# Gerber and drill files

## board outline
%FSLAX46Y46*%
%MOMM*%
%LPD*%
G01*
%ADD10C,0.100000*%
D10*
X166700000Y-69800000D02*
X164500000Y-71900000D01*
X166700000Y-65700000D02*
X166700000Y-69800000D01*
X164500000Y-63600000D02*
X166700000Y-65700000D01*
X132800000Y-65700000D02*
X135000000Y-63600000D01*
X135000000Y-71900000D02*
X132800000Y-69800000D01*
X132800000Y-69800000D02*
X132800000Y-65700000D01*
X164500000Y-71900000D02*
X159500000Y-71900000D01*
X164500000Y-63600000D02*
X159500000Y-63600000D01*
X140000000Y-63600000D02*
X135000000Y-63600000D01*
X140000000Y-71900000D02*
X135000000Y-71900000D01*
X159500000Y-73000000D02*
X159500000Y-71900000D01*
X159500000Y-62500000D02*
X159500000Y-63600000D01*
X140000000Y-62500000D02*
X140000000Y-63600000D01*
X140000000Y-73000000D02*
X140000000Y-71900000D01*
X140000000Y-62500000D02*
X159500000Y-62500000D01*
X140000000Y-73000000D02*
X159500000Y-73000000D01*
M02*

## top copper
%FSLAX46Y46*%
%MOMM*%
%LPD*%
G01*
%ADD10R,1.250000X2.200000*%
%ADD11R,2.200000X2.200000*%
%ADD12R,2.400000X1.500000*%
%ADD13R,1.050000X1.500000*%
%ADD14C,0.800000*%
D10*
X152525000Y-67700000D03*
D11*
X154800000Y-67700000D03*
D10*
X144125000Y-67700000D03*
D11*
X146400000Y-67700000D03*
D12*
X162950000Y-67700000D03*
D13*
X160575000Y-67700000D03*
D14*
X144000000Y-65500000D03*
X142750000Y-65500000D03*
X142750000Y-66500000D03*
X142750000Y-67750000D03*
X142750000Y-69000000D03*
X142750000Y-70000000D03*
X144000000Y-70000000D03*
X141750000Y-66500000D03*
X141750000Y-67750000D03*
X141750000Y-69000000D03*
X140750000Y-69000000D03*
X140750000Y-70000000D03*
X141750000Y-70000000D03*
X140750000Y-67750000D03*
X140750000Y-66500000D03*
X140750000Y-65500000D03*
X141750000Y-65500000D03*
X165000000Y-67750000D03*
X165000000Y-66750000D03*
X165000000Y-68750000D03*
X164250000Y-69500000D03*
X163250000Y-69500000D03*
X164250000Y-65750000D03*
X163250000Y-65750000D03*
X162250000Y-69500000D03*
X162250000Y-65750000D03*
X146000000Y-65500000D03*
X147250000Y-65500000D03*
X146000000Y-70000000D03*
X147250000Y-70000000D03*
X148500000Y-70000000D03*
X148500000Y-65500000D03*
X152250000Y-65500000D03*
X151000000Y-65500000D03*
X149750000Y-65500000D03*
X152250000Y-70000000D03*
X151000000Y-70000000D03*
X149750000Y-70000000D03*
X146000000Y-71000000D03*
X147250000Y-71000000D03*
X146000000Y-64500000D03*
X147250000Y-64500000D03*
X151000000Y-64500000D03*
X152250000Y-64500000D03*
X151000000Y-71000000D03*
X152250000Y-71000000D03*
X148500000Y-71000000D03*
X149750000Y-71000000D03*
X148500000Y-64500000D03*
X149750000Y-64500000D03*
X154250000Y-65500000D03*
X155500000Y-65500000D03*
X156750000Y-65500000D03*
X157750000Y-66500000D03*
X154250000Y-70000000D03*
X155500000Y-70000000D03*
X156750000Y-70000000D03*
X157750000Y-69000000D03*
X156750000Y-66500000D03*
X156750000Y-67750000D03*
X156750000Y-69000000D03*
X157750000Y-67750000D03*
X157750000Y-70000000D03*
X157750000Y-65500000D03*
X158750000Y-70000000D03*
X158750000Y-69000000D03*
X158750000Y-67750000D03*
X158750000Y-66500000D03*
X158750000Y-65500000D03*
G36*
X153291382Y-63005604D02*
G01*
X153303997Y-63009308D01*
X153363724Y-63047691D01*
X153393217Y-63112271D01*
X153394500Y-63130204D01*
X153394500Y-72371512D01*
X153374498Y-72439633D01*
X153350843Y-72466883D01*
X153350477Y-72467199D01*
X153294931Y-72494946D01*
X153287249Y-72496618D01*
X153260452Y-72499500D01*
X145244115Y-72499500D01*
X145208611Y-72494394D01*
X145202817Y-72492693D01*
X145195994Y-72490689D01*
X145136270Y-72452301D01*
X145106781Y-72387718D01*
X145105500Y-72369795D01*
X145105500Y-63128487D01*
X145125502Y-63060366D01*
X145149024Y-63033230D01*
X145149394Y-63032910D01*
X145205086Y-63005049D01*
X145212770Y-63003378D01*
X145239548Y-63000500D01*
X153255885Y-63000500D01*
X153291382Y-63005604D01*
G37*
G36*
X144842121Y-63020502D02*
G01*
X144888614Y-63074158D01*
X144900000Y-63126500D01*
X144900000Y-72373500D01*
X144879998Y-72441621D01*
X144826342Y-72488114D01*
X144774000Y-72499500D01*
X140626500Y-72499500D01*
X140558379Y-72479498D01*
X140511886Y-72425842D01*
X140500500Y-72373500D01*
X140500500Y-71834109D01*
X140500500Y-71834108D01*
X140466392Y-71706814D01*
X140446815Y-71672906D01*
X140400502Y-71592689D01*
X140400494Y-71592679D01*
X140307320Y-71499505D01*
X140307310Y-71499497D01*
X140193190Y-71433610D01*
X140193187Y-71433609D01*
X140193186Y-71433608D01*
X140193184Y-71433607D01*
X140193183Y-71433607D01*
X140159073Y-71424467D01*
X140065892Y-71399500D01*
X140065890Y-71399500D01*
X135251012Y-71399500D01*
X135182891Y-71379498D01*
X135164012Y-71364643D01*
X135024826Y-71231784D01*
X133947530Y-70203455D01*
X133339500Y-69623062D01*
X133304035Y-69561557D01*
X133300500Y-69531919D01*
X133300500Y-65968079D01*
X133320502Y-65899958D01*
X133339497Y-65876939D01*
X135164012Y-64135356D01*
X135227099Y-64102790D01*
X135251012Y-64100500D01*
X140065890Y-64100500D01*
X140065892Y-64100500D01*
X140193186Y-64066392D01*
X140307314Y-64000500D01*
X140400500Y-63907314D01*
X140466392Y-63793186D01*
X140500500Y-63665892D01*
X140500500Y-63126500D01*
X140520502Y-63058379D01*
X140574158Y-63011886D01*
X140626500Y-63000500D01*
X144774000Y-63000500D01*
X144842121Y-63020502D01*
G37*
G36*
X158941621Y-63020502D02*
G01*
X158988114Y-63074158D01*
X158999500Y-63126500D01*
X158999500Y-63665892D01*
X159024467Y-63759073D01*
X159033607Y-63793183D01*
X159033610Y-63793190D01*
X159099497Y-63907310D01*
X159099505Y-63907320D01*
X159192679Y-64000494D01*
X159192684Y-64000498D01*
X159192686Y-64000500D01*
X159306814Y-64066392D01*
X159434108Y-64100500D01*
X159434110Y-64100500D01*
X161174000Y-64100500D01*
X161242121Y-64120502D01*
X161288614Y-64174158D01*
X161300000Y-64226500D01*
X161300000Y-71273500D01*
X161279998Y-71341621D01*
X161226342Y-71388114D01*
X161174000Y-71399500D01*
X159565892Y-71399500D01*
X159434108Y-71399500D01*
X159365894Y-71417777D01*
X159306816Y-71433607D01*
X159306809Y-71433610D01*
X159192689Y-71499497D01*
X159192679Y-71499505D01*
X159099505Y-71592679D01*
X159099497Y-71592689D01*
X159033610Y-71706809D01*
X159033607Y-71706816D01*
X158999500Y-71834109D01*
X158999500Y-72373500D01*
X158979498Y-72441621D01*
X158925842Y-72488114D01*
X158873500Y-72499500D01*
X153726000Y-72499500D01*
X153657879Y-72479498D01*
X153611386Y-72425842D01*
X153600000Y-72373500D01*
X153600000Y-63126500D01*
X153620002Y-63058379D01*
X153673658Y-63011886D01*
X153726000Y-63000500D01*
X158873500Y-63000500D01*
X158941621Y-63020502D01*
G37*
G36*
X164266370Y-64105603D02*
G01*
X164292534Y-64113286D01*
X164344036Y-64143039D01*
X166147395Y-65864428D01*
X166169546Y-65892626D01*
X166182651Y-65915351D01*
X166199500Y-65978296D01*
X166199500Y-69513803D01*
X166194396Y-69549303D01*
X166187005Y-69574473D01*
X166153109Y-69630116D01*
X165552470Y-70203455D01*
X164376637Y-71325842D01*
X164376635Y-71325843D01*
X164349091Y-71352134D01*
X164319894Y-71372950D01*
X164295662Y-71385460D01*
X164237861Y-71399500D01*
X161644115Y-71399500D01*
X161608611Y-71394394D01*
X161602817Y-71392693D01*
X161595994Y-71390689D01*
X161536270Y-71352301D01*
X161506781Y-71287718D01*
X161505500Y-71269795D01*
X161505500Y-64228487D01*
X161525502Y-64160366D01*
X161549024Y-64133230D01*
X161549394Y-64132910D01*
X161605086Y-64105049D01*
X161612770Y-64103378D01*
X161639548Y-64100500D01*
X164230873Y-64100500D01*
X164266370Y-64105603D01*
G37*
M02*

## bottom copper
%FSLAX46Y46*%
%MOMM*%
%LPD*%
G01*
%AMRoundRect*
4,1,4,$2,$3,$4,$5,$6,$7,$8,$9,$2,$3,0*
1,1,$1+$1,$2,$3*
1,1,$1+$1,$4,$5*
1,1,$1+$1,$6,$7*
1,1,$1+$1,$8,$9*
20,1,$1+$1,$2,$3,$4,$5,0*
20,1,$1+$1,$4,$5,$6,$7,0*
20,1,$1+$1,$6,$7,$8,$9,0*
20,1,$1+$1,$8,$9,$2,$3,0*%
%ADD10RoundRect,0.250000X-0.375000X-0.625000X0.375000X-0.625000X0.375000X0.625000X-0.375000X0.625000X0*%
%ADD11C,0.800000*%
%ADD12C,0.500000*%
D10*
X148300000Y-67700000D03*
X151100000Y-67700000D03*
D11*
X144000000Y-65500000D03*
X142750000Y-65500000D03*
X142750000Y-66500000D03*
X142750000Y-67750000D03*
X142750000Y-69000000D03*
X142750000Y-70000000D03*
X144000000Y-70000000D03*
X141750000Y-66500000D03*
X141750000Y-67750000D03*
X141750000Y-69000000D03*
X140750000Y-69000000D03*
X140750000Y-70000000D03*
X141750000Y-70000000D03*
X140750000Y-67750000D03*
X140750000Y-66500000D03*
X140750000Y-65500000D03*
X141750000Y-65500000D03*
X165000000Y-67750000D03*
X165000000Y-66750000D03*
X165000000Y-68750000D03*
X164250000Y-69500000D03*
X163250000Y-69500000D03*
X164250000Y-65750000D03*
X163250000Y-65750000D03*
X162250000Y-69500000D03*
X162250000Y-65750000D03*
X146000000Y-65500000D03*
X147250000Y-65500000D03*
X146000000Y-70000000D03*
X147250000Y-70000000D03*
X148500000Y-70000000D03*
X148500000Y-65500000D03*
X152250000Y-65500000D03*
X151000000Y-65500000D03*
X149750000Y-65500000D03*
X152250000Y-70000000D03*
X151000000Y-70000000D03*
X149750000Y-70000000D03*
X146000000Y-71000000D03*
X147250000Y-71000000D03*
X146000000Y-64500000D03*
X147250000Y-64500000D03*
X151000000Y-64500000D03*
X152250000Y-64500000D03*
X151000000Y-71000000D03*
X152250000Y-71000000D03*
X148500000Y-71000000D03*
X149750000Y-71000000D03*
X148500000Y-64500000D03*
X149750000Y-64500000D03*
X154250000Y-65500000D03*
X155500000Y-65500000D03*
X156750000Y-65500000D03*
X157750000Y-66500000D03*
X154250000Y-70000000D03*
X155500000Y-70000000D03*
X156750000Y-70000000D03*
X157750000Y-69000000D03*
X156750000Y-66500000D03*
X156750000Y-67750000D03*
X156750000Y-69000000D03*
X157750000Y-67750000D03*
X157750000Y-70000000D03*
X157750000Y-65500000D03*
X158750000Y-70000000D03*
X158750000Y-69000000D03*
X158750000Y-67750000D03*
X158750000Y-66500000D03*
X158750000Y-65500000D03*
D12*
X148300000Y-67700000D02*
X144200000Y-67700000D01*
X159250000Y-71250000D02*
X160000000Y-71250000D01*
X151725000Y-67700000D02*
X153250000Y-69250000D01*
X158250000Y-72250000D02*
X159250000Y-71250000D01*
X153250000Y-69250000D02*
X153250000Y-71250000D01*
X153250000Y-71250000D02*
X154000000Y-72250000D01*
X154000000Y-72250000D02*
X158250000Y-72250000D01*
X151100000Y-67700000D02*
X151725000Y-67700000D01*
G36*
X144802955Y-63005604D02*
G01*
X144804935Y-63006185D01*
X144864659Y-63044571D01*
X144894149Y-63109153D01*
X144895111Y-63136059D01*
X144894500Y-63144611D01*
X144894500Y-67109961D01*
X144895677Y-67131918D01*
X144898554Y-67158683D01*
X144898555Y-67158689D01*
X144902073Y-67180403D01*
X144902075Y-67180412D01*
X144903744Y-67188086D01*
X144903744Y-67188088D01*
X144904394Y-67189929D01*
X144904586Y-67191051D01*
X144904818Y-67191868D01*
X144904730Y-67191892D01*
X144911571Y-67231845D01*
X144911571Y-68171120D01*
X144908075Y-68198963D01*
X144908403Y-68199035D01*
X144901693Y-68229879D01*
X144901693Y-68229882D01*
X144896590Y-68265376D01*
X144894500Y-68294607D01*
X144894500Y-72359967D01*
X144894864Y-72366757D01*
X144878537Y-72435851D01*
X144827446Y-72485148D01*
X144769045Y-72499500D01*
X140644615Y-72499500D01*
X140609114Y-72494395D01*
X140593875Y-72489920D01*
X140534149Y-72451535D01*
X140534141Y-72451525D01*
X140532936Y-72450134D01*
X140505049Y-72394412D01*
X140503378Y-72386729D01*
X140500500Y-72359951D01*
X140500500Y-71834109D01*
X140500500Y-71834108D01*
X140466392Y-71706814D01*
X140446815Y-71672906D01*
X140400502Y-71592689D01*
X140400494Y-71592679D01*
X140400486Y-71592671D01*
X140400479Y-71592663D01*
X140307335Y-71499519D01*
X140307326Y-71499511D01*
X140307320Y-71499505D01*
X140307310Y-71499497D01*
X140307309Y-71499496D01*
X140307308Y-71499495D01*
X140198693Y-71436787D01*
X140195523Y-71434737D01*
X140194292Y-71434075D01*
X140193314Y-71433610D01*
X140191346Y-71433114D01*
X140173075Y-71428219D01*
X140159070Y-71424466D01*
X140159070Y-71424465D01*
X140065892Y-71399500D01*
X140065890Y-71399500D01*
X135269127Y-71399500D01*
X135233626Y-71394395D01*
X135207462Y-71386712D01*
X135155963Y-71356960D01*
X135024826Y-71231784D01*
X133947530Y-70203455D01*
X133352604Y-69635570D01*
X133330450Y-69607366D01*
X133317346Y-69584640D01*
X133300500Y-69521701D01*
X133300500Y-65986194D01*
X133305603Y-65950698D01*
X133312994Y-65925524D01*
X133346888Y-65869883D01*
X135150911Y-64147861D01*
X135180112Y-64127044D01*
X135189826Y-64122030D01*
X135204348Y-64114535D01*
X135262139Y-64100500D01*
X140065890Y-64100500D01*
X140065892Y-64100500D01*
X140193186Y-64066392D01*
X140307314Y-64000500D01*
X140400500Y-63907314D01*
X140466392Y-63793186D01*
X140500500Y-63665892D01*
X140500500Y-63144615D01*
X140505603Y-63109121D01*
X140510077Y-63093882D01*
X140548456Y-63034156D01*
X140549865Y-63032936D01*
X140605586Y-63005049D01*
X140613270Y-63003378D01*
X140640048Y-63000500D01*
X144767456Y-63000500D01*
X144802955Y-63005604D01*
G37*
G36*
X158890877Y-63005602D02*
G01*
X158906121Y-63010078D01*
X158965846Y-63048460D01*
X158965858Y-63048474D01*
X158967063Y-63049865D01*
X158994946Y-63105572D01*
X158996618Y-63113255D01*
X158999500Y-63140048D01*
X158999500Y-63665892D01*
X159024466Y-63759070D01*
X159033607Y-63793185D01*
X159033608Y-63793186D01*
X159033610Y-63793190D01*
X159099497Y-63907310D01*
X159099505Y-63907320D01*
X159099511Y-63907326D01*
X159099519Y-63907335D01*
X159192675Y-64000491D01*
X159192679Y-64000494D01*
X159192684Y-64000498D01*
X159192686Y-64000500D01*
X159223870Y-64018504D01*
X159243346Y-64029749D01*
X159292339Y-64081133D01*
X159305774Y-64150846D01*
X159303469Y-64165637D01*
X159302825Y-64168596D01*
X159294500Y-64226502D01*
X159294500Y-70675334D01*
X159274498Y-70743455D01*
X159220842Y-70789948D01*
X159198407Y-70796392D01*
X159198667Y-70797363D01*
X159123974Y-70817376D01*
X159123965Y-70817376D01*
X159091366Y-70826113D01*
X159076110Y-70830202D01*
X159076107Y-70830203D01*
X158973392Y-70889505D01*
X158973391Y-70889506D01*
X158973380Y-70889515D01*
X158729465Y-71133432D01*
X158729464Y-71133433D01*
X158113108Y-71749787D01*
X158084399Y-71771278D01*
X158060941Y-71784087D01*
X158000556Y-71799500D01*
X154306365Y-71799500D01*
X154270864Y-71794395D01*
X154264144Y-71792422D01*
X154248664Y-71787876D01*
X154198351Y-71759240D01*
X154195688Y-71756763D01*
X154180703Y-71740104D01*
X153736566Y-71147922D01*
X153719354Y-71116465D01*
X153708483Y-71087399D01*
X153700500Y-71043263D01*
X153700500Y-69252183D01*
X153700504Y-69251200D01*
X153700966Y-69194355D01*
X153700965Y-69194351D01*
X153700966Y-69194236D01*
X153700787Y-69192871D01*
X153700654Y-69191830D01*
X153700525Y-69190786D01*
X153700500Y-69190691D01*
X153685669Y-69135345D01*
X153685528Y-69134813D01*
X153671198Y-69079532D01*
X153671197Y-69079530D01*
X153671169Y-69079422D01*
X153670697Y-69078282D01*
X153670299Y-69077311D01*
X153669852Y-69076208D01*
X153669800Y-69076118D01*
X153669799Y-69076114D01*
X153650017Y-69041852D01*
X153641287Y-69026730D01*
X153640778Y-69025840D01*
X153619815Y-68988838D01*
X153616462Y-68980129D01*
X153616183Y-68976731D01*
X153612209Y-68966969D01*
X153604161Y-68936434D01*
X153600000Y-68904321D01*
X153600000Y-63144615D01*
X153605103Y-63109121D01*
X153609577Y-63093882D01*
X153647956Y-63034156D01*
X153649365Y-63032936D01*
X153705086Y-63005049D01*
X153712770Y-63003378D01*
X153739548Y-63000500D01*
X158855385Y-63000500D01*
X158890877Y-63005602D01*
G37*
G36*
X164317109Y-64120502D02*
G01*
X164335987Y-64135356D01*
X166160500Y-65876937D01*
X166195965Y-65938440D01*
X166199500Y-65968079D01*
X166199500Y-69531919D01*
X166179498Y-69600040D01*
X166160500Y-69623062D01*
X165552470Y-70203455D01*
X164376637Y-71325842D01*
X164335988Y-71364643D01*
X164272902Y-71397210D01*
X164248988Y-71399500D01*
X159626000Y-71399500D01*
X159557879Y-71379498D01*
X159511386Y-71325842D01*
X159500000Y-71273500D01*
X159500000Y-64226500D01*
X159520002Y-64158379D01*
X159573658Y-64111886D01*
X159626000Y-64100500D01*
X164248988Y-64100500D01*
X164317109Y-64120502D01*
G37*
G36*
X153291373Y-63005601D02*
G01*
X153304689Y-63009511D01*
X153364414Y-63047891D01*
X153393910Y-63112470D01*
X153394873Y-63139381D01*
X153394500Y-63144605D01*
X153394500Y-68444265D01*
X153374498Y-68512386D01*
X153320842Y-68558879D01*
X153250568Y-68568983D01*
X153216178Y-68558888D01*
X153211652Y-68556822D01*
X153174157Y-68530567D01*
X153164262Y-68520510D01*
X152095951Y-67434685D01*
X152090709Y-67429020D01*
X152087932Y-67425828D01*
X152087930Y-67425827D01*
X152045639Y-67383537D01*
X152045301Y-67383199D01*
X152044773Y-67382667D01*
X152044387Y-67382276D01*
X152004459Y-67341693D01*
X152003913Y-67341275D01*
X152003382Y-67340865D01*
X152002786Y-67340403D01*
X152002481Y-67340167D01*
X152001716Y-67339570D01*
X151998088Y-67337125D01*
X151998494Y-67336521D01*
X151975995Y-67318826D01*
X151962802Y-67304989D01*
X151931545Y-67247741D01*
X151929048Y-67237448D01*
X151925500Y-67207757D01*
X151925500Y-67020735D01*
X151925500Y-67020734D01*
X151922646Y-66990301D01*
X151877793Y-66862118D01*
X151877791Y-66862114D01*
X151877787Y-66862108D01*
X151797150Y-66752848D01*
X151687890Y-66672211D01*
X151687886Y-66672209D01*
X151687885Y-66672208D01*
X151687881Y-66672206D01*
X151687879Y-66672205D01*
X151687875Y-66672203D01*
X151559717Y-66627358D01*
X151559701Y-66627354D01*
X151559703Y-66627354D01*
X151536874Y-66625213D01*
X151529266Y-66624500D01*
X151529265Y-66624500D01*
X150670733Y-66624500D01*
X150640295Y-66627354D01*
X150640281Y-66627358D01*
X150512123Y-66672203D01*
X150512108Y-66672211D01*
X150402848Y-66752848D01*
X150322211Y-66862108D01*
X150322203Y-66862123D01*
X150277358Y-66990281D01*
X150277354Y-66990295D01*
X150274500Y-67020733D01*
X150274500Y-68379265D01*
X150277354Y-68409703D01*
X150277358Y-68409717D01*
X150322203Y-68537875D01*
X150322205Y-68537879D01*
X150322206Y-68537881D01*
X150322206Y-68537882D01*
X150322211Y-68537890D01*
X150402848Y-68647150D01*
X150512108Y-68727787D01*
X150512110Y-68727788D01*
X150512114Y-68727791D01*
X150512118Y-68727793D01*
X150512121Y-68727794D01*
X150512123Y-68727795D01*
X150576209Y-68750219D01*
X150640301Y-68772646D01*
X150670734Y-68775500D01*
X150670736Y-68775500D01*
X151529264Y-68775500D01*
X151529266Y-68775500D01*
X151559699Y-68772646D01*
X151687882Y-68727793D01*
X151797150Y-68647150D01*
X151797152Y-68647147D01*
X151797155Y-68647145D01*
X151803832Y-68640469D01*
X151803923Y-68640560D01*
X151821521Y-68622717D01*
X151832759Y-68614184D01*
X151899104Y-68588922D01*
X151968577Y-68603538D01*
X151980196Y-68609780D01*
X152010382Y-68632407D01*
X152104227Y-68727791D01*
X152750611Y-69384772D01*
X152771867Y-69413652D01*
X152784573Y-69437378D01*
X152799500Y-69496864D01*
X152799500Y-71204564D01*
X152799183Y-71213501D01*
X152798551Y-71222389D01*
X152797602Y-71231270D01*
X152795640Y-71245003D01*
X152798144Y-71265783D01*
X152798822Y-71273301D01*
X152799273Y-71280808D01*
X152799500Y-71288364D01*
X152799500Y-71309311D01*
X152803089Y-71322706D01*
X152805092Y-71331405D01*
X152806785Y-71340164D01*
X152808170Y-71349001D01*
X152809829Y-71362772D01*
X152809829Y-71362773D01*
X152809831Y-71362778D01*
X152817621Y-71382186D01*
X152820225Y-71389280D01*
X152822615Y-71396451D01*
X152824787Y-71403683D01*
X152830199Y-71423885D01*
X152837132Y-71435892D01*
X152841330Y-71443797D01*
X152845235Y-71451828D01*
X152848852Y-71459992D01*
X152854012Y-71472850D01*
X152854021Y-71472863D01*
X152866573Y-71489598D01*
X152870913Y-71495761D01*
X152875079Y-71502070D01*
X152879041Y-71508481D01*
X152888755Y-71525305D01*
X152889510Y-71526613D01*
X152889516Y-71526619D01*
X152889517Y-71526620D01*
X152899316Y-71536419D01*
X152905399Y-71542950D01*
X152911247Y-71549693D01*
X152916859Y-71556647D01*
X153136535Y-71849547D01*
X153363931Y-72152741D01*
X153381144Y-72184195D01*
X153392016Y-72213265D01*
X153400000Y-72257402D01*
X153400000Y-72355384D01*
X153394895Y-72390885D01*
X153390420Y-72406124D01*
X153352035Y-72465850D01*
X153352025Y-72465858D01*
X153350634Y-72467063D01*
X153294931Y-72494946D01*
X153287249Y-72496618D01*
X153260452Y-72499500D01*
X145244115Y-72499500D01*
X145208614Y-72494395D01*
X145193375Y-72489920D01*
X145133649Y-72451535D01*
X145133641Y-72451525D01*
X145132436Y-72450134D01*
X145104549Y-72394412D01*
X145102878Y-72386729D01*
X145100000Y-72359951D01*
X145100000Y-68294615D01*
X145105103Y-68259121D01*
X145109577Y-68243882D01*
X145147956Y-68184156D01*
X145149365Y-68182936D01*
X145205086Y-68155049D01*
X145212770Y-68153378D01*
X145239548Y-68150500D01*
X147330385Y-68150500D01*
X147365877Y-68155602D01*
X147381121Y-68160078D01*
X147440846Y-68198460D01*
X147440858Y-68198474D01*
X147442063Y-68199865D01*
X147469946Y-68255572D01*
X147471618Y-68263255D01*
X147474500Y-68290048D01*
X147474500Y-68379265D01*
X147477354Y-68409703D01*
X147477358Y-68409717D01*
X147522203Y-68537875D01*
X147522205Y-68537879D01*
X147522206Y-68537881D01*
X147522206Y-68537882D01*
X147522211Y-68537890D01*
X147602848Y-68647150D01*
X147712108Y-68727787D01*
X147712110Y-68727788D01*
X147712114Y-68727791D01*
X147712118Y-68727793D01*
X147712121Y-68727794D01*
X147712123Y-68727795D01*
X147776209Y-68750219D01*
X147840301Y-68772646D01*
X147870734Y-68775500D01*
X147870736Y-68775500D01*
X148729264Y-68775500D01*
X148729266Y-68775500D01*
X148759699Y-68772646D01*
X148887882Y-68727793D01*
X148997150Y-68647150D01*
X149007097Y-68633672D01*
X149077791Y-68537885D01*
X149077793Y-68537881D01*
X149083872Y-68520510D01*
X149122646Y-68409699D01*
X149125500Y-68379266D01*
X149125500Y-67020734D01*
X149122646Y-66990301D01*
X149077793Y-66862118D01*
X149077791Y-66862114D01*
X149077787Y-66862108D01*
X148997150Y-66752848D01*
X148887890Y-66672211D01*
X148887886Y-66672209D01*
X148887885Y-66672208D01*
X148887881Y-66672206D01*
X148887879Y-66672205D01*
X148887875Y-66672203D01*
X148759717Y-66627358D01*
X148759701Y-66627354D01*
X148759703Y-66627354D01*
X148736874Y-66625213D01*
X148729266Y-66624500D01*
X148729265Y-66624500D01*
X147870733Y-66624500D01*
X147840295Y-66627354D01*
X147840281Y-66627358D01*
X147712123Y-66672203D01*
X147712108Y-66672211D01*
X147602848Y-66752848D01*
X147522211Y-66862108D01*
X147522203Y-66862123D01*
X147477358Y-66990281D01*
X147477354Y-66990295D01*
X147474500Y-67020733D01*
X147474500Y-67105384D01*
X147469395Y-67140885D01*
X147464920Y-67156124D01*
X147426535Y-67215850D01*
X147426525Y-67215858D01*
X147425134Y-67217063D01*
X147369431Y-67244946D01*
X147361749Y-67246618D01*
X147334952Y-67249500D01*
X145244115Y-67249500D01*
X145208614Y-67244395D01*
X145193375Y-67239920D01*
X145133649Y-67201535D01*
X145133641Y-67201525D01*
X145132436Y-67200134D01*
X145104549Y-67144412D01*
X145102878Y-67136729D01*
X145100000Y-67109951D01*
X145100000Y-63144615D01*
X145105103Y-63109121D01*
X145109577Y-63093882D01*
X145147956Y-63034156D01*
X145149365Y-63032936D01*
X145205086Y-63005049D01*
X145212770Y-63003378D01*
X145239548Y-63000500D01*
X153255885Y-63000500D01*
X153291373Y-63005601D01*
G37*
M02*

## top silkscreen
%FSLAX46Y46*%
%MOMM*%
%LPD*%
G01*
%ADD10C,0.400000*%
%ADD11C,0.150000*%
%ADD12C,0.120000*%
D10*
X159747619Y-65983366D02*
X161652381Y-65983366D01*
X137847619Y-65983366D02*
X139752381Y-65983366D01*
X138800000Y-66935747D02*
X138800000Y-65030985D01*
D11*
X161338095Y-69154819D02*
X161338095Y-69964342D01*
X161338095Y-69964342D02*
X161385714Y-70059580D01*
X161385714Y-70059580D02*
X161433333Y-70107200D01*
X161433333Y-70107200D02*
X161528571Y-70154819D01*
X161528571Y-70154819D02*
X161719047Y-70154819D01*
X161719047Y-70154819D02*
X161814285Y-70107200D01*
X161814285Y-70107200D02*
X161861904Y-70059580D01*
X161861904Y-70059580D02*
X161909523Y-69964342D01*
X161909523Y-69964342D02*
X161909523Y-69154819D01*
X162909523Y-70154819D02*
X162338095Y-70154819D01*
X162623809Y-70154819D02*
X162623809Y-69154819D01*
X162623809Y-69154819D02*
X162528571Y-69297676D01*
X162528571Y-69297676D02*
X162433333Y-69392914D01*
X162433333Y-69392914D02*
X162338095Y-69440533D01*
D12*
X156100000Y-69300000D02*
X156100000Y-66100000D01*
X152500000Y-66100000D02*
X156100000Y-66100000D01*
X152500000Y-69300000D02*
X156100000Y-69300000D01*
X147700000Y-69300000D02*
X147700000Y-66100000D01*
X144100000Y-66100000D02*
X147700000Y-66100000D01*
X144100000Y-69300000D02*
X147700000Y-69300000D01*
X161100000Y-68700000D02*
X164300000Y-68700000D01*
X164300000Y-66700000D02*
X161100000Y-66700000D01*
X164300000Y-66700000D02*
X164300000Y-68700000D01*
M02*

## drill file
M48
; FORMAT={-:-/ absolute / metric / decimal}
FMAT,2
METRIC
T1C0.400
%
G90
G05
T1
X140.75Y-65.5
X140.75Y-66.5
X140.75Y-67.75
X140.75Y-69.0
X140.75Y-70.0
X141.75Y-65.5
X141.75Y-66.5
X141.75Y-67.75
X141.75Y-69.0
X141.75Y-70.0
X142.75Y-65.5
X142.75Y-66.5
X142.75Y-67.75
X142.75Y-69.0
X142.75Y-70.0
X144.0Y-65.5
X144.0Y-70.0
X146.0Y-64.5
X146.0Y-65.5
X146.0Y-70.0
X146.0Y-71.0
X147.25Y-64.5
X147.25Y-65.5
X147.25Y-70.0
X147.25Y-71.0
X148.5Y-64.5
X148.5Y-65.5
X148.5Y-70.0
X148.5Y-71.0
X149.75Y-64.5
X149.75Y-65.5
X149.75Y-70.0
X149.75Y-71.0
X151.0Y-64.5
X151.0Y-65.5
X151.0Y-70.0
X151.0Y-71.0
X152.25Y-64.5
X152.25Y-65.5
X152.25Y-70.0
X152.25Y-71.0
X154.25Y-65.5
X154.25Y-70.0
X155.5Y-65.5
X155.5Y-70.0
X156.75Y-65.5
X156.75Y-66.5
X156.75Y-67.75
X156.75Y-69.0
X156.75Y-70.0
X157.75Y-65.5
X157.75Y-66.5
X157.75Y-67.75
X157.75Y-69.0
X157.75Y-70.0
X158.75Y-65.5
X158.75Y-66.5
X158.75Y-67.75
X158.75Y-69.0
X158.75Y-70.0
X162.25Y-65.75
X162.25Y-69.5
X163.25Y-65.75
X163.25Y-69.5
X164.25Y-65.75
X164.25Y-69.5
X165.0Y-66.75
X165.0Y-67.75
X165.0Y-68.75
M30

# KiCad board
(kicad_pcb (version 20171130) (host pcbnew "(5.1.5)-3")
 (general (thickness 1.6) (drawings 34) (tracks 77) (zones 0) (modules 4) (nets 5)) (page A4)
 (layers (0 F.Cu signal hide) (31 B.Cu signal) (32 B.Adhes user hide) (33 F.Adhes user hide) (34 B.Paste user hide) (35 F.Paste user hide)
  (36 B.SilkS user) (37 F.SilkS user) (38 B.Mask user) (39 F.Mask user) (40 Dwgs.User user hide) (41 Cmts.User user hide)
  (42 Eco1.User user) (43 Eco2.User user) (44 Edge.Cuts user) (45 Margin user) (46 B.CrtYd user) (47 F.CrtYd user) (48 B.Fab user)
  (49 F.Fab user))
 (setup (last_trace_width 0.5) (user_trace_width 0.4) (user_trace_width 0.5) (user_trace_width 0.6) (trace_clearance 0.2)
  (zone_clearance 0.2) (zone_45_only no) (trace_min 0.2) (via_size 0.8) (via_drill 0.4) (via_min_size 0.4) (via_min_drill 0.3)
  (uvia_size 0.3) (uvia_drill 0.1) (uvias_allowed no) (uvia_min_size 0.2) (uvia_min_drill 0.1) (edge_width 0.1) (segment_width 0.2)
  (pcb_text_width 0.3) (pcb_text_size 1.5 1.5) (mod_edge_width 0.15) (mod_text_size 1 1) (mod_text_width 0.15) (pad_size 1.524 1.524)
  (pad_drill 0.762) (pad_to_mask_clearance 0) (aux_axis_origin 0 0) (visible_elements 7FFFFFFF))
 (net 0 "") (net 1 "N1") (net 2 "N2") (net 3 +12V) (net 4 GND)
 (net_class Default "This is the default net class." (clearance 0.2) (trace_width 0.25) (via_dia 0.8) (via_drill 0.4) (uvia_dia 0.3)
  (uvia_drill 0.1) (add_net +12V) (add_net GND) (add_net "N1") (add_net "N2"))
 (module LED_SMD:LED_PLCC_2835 (layer F.Cu) (at 153.9 67.7 180)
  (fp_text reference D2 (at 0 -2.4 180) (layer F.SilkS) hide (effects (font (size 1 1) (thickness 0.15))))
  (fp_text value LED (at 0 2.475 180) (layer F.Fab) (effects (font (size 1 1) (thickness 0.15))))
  (fp_line (start -2.2 -1.6) (end -2.2 1.6) (layer F.SilkS) (width 0.12))
  (fp_line (start 1.4 1.6) (end -2.2 1.6) (layer F.SilkS) (width 0.12))
  (fp_line (start 1.4 -1.6) (end -2.2 -1.6) (layer F.SilkS) (width 0.12))
  (pad 2 smd rect (at 1.375 0 180) (size 1.25 2.2) (layers F.Cu F.Paste F.Mask) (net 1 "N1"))
  (pad 1 smd rect (at -0.9 0 180) (size 2.2 2.2) (layers F.Cu F.Paste F.Mask) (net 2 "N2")))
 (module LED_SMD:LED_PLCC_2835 (layer F.Cu) (at 145.5 67.7 180)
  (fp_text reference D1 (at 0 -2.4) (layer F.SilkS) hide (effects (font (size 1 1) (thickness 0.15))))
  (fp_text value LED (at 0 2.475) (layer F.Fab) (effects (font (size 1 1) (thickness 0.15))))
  (fp_line (start -2.2 -1.6) (end -2.2 1.6) (layer F.SilkS) (width 0.12))
  (fp_line (start 1.4 1.6) (end -2.2 1.6) (layer F.SilkS) (width 0.12))
  (fp_line (start 1.4 -1.6) (end -2.2 -1.6) (layer F.SilkS) (width 0.12))
  (pad 2 smd rect (at 1.375 0 180) (size 1.25 2.2) (layers F.Cu F.Paste F.Mask) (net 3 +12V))
  (pad 1 smd rect (at -0.9 0 180) (size 2.2 2.2) (layers F.Cu F.Paste F.Mask) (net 1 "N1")))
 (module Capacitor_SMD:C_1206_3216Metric (layer B.Cu) (at 149.7 67.7)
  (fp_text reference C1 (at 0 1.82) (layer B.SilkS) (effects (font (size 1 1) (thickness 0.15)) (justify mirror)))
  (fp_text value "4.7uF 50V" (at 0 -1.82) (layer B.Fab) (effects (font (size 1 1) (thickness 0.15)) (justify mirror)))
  (pad 1 smd roundrect (at -1.4 0) (size 1.25 1.75) (layers B.Cu B.Paste B.Mask) (roundrect_rratio 0.2) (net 3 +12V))
  (pad 2 smd roundrect (at 1.4 0) (size 1.25 1.75) (layers B.Cu B.Paste B.Mask) (roundrect_rratio 0.2) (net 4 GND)))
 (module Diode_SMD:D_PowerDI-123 (layer F.Cu) (at 162.1 67.7 180)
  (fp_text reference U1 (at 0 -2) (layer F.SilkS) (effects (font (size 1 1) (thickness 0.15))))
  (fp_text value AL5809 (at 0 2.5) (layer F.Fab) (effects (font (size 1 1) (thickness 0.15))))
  (fp_line (start 1 -1) (end -2.2 -1) (layer F.SilkS) (width 0.12))
  (fp_line (start -2.2 1) (end 1 1) (layer F.SilkS) (width 0.12))
  (fp_line (start -2.2 1) (end -2.2 -1) (layer F.SilkS) (width 0.12))
  (pad 1 smd rect (at -0.85 0) (size 2.4 1.5) (layers F.Cu F.Paste F.Mask) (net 4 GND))
  (pad 2 smd rect (at 1.525 0) (size 1.05 1.5) (layers F.Cu F.Paste F.Mask) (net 2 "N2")))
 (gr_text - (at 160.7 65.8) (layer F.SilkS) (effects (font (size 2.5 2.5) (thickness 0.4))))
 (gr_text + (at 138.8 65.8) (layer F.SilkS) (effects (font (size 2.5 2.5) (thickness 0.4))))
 (gr_line (start 166.7 69.8) (end 164.5 71.9) (layer Edge.Cuts) (width 0.1))
 (gr_line (start 166.7 65.7) (end 166.7 69.8) (layer Edge.Cuts) (width 0.1))
 (gr_line (start 164.5 63.6) (end 166.7 65.7) (layer Edge.Cuts) (width 0.1))
 (gr_line (start 132.8 65.7) (end 135 63.6) (layer Edge.Cuts) (width 0.1))
 (gr_line (start 135 71.9) (end 132.8 69.8) (layer Edge.Cuts) (width 0.1))
 (gr_line (start 132.8 69.8) (end 132.8 65.7) (layer Edge.Cuts) (width 0.1))
 (gr_line (start 164.5 71.9) (end 159.5 71.9) (layer Edge.Cuts) (width 0.1))
 (gr_line (start 164.5 63.6) (end 159.5 63.6) (layer Edge.Cuts) (width 0.1))
 (gr_line (start 140 63.6) (end 135 63.6) (layer Edge.Cuts) (width 0.1))
 (gr_line (start 140 71.9) (end 135 71.9) (layer Edge.Cuts) (width 0.1))
 (gr_line (start 159.5 73) (end 159.5 71.9) (layer Edge.Cuts) (width 0.1))
 (gr_line (start 159.5 62.5) (end 159.5 63.6) (layer Edge.Cuts) (width 0.1))
 (gr_line (start 140 62.5) (end 140 63.6) (layer Edge.Cuts) (width 0.1))
 (gr_line (start 140 73) (end 140 71.9) (layer Edge.Cuts) (width 0.1))
 (gr_line (start 140 62.5) (end 159.5 62.5) (layer Edge.Cuts) (width 0.1))
 (gr_line (start 140 73) (end 159.5 73) (layer Edge.Cuts) (width 0.1))
 (via (at 144 65.5) (size 0.8) (drill 0.4) (layers F.Cu B.Cu) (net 3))
 (via (at 142.75 65.5) (size 0.8) (drill 0.4) (layers F.Cu B.Cu) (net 3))
 (via (at 142.75 66.5) (size 0.8) (drill 0.4) (layers F.Cu B.Cu) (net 3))
 (via (at 142.75 67.75) (size 0.8) (drill 0.4) (layers F.Cu B.Cu) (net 3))
 (via (at 142.75 69) (size 0.8) (drill 0.4) (layers F.Cu B.Cu) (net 3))
 (via (at 142.75 70) (size 0.8) (drill 0.4) (layers F.Cu B.Cu) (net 3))
 (via (at 144 70) (size 0.8) (drill 0.4) (layers F.Cu B.Cu) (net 3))
 (via (at 141.75 66.5) (size 0.8) (drill 0.4) (layers F.Cu B.Cu) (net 3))
 (via (at 141.75 67.75) (size 0.8) (drill 0.4) (layers F.Cu B.Cu) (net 3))
 (via (at 141.75 69) (size 0.8) (drill 0.4) (layers F.Cu B.Cu) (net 3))
 (segment (start 148.3 67.7) (end 144.2 67.7) (width 0.5) (layer B.Cu) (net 3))
 (via (at 140.75 69) (size 0.8) (drill 0.4) (layers F.Cu B.Cu) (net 3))
 (via (at 140.75 70) (size 0.8) (drill 0.4) (layers F.Cu B.Cu) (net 3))
 (via (at 141.75 70) (size 0.8) (drill 0.4) (layers F.Cu B.Cu) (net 3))
 (via (at 140.75 67.75) (size 0.8) (drill 0.4) (layers F.Cu B.Cu) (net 3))
 (via (at 140.75 66.5) (size 0.8) (drill 0.4) (layers F.Cu B.Cu) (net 3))
 (via (at 140.75 65.5) (size 0.8) (drill 0.4) (layers F.Cu B.Cu) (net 3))
 (via (at 141.75 65.5) (size 0.8) (drill 0.4) (layers F.Cu B.Cu) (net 3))
 (via (at 165 67.75) (size 0.8) (drill 0.4) (layers F.Cu B.Cu) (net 4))
 (via (at 165 66.75) (size 0.8) (drill 0.4) (layers F.Cu B.Cu) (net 4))
 (via (at 165 68.75) (size 0.8) (drill 0.4) (layers F.Cu B.Cu) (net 4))
 (via (at 164.25 69.5) (size 0.8) (drill 0.4) (layers F.Cu B.Cu) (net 4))
 (via (at 163.25 69.5) (size 0.8) (drill 0.4) (layers F.Cu B.Cu) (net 4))
 (via (at 164.25 65.75) (size 0.8) (drill 0.4) (layers F.Cu B.Cu) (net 4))
 (via (at 163.25 65.75) (size 0.8) (drill 0.4) (layers F.Cu B.Cu) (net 4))
 (via (at 162.25 69.5) (size 0.8) (drill 0.4) (layers F.Cu B.Cu) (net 4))
 (via (at 162.25 65.75) (size 0.8) (drill 0.4) (layers F.Cu B.Cu) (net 4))
 (segment (start 159.25 71.25) (end 160 71.25) (width 0.5) (layer B.Cu) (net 4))
 (segment (start 151.725 67.7) (end 153.25 69.25) (width 0.5) (layer B.Cu) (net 4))
 (segment (start 158.25 72.25) (end 159.25 71.25) (width 0.5) (layer B.Cu) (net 4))
 (segment (start 153.25 69.25) (end 153.25 71.25) (width 0.5) (layer B.Cu) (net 4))
 (segment (start 153.25 71.25) (end 154 72.25) (width 0.5) (layer B.Cu) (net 4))
 (segment (start 154 72.25) (end 158.25 72.25) (width 0.5) (layer B.Cu) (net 4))
 (segment (start 151.1 67.7) (end 151.725 67.7) (width 0.5) (layer B.Cu) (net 4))
 (via (at 146 65.5) (size 0.8) (drill 0.4) (layers F.Cu B.Cu) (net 1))
 (via (at 147.25 65.5) (size 0.8) (drill 0.4) (layers F.Cu B.Cu) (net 1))
 (via (at 146 70) (size 0.8) (drill 0.4) (layers F.Cu B.Cu) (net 1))
 (via (at 147.25 70) (size 0.8) (drill 0.4) (layers F.Cu B.Cu) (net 1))
 (via (at 148.5 70) (size 0.8) (drill 0.4) (layers F.Cu B.Cu) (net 1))
 (via (at 148.5 65.5) (size 0.8) (drill 0.4) (layers F.Cu B.Cu) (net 1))
 (via (at 152.25 65.5) (size 0.8) (drill 0.4) (layers F.Cu B.Cu) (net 1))
 (via (at 151 65.5) (size 0.8) (drill 0.4) (layers F.Cu B.Cu) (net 1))
 (via (at 149.75 65.5) (size 0.8) (drill 0.4) (layers F.Cu B.Cu) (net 1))
 (via (at 152.25 70) (size 0.8) (drill 0.4) (layers F.Cu B.Cu) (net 1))
 (via (at 151 70) (size 0.8) (drill 0.4) (layers F.Cu B.Cu) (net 1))
 (via (at 149.75 70) (size 0.8) (drill 0.4) (layers F.Cu B.Cu) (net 1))
 (via (at 146 71) (size 0.8) (drill 0.4) (layers F.Cu B.Cu) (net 1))
 (via (at 147.25 71) (size 0.8) (drill 0.4) (layers F.Cu B.Cu) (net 1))
 (via (at 146 64.5) (size 0.8) (drill 0.4) (layers F.Cu B.Cu) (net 1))
 (via (at 147.25 64.5) (size 0.8) (drill 0.4) (layers F.Cu B.Cu) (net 1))
 (via (at 151 64.5) (size 0.8) (drill 0.4) (layers F.Cu B.Cu) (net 1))
 (via (at 152.25 64.5) (size 0.8) (drill 0.4) (layers F.Cu B.Cu) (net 1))
 (via (at 151 71) (size 0.8) (drill 0.4) (layers F.Cu B.Cu) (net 1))
 (via (at 152.25 71) (size 0.8) (drill 0.4) (layers F.Cu B.Cu) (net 1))
 (via (at 148.5 71) (size 0.8) (drill 0.4) (layers F.Cu B.Cu) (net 1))
 (via (at 149.75 71) (size 0.8) (drill 0.4) (layers F.Cu B.Cu) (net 1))
 (via (at 148.5 64.5) (size 0.8) (drill 0.4) (layers F.Cu B.Cu) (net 1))
 (via (at 149.75 64.5) (size 0.8) (drill 0.4) (layers F.Cu B.Cu) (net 1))
 (via (at 154.25 65.5) (size 0.8) (drill 0.4) (layers F.Cu B.Cu) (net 2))
 (via (at 155.5 65.5) (size 0.8) (drill 0.4) (layers F.Cu B.Cu) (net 2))
 (via (at 156.75 65.5) (size 0.8) (drill 0.4) (layers F.Cu B.Cu) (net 2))
 (via (at 157.75 66.5) (size 0.8) (drill 0.4) (layers F.Cu B.Cu) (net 2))
 (via (at 154.25 70) (size 0.8) (drill 0.4) (layers F.Cu B.Cu) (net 2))
 (via (at 155.5 70) (size 0.8) (drill 0.4) (layers F.Cu B.Cu) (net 2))
 (via (at 156.75 70) (size 0.8) (drill 0.4) (layers F.Cu B.Cu) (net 2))
 (via (at 157.75 69) (size 0.8) (drill 0.4) (layers F.Cu B.Cu) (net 2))
 (via (at 156.75 66.5) (size 0.8) (drill 0.4) (layers F.Cu B.Cu) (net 2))
 (via (at 156.75 67.75) (size 0.8) (drill 0.4) (layers F.Cu B.Cu) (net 2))
 (via (at 156.75 69) (size 0.8) (drill 0.4) (layers F.Cu B.Cu) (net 2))
 (via (at 157.75 67.75) (size 0.8) (drill 0.4) (layers F.Cu B.Cu) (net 2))
 (via (at 157.75 70) (size 0.8) (drill 0.4) (layers F.Cu B.Cu) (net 2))
 (via (at 157.75 65.5) (size 0.8) (drill 0.4) (layers F.Cu B.Cu) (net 2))
 (via (at 158.75 70) (size 0.8) (drill 0.4) (layers F.Cu B.Cu) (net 2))
 (via (at 158.75 69) (size 0.8) (drill 0.4) (layers F.Cu B.Cu) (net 2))
 (via (at 158.75 67.75) (size 0.8) (drill 0.4) (layers F.Cu B.Cu) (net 2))
 (via (at 158.75 66.5) (size 0.8) (drill 0.4) (layers F.Cu B.Cu) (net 2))
 (via (at 158.75 65.5) (size 0.8) (drill 0.4) (layers F.Cu B.Cu) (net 2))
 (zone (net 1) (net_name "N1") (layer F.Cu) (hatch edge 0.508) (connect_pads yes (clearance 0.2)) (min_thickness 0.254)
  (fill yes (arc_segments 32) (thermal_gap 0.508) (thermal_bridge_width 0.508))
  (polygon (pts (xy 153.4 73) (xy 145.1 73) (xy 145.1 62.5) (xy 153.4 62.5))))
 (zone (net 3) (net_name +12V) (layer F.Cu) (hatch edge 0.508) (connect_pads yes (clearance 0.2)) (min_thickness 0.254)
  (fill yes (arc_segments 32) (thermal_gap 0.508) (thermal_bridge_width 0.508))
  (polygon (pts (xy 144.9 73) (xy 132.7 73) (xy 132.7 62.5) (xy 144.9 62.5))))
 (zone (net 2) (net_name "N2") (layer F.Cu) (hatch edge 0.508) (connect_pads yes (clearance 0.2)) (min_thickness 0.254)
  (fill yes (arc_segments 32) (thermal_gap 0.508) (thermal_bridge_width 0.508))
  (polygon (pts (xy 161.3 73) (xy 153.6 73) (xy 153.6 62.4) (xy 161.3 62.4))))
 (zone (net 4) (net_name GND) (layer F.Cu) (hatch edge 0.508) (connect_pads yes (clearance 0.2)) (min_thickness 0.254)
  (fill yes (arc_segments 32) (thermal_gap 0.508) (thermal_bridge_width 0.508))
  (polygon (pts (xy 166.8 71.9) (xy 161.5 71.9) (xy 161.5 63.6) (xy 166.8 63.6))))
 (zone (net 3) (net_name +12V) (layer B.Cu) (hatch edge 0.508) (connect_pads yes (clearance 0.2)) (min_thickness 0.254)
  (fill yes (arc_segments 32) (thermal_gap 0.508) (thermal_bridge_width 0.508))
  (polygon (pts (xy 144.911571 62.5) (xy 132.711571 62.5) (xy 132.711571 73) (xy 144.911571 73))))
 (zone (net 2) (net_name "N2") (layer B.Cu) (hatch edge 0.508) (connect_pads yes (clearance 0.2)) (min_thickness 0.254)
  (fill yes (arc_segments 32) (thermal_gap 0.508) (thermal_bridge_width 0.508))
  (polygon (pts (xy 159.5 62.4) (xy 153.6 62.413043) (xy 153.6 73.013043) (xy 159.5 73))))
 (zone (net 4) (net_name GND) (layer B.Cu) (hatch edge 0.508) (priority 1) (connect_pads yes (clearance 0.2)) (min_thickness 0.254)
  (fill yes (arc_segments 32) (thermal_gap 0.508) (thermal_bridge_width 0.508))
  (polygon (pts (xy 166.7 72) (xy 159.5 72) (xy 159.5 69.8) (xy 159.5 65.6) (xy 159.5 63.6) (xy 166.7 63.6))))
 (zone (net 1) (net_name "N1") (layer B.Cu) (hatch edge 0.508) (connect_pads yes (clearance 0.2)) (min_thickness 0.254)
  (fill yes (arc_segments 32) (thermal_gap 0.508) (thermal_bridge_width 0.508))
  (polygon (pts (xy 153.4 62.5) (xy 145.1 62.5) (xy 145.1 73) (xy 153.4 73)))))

